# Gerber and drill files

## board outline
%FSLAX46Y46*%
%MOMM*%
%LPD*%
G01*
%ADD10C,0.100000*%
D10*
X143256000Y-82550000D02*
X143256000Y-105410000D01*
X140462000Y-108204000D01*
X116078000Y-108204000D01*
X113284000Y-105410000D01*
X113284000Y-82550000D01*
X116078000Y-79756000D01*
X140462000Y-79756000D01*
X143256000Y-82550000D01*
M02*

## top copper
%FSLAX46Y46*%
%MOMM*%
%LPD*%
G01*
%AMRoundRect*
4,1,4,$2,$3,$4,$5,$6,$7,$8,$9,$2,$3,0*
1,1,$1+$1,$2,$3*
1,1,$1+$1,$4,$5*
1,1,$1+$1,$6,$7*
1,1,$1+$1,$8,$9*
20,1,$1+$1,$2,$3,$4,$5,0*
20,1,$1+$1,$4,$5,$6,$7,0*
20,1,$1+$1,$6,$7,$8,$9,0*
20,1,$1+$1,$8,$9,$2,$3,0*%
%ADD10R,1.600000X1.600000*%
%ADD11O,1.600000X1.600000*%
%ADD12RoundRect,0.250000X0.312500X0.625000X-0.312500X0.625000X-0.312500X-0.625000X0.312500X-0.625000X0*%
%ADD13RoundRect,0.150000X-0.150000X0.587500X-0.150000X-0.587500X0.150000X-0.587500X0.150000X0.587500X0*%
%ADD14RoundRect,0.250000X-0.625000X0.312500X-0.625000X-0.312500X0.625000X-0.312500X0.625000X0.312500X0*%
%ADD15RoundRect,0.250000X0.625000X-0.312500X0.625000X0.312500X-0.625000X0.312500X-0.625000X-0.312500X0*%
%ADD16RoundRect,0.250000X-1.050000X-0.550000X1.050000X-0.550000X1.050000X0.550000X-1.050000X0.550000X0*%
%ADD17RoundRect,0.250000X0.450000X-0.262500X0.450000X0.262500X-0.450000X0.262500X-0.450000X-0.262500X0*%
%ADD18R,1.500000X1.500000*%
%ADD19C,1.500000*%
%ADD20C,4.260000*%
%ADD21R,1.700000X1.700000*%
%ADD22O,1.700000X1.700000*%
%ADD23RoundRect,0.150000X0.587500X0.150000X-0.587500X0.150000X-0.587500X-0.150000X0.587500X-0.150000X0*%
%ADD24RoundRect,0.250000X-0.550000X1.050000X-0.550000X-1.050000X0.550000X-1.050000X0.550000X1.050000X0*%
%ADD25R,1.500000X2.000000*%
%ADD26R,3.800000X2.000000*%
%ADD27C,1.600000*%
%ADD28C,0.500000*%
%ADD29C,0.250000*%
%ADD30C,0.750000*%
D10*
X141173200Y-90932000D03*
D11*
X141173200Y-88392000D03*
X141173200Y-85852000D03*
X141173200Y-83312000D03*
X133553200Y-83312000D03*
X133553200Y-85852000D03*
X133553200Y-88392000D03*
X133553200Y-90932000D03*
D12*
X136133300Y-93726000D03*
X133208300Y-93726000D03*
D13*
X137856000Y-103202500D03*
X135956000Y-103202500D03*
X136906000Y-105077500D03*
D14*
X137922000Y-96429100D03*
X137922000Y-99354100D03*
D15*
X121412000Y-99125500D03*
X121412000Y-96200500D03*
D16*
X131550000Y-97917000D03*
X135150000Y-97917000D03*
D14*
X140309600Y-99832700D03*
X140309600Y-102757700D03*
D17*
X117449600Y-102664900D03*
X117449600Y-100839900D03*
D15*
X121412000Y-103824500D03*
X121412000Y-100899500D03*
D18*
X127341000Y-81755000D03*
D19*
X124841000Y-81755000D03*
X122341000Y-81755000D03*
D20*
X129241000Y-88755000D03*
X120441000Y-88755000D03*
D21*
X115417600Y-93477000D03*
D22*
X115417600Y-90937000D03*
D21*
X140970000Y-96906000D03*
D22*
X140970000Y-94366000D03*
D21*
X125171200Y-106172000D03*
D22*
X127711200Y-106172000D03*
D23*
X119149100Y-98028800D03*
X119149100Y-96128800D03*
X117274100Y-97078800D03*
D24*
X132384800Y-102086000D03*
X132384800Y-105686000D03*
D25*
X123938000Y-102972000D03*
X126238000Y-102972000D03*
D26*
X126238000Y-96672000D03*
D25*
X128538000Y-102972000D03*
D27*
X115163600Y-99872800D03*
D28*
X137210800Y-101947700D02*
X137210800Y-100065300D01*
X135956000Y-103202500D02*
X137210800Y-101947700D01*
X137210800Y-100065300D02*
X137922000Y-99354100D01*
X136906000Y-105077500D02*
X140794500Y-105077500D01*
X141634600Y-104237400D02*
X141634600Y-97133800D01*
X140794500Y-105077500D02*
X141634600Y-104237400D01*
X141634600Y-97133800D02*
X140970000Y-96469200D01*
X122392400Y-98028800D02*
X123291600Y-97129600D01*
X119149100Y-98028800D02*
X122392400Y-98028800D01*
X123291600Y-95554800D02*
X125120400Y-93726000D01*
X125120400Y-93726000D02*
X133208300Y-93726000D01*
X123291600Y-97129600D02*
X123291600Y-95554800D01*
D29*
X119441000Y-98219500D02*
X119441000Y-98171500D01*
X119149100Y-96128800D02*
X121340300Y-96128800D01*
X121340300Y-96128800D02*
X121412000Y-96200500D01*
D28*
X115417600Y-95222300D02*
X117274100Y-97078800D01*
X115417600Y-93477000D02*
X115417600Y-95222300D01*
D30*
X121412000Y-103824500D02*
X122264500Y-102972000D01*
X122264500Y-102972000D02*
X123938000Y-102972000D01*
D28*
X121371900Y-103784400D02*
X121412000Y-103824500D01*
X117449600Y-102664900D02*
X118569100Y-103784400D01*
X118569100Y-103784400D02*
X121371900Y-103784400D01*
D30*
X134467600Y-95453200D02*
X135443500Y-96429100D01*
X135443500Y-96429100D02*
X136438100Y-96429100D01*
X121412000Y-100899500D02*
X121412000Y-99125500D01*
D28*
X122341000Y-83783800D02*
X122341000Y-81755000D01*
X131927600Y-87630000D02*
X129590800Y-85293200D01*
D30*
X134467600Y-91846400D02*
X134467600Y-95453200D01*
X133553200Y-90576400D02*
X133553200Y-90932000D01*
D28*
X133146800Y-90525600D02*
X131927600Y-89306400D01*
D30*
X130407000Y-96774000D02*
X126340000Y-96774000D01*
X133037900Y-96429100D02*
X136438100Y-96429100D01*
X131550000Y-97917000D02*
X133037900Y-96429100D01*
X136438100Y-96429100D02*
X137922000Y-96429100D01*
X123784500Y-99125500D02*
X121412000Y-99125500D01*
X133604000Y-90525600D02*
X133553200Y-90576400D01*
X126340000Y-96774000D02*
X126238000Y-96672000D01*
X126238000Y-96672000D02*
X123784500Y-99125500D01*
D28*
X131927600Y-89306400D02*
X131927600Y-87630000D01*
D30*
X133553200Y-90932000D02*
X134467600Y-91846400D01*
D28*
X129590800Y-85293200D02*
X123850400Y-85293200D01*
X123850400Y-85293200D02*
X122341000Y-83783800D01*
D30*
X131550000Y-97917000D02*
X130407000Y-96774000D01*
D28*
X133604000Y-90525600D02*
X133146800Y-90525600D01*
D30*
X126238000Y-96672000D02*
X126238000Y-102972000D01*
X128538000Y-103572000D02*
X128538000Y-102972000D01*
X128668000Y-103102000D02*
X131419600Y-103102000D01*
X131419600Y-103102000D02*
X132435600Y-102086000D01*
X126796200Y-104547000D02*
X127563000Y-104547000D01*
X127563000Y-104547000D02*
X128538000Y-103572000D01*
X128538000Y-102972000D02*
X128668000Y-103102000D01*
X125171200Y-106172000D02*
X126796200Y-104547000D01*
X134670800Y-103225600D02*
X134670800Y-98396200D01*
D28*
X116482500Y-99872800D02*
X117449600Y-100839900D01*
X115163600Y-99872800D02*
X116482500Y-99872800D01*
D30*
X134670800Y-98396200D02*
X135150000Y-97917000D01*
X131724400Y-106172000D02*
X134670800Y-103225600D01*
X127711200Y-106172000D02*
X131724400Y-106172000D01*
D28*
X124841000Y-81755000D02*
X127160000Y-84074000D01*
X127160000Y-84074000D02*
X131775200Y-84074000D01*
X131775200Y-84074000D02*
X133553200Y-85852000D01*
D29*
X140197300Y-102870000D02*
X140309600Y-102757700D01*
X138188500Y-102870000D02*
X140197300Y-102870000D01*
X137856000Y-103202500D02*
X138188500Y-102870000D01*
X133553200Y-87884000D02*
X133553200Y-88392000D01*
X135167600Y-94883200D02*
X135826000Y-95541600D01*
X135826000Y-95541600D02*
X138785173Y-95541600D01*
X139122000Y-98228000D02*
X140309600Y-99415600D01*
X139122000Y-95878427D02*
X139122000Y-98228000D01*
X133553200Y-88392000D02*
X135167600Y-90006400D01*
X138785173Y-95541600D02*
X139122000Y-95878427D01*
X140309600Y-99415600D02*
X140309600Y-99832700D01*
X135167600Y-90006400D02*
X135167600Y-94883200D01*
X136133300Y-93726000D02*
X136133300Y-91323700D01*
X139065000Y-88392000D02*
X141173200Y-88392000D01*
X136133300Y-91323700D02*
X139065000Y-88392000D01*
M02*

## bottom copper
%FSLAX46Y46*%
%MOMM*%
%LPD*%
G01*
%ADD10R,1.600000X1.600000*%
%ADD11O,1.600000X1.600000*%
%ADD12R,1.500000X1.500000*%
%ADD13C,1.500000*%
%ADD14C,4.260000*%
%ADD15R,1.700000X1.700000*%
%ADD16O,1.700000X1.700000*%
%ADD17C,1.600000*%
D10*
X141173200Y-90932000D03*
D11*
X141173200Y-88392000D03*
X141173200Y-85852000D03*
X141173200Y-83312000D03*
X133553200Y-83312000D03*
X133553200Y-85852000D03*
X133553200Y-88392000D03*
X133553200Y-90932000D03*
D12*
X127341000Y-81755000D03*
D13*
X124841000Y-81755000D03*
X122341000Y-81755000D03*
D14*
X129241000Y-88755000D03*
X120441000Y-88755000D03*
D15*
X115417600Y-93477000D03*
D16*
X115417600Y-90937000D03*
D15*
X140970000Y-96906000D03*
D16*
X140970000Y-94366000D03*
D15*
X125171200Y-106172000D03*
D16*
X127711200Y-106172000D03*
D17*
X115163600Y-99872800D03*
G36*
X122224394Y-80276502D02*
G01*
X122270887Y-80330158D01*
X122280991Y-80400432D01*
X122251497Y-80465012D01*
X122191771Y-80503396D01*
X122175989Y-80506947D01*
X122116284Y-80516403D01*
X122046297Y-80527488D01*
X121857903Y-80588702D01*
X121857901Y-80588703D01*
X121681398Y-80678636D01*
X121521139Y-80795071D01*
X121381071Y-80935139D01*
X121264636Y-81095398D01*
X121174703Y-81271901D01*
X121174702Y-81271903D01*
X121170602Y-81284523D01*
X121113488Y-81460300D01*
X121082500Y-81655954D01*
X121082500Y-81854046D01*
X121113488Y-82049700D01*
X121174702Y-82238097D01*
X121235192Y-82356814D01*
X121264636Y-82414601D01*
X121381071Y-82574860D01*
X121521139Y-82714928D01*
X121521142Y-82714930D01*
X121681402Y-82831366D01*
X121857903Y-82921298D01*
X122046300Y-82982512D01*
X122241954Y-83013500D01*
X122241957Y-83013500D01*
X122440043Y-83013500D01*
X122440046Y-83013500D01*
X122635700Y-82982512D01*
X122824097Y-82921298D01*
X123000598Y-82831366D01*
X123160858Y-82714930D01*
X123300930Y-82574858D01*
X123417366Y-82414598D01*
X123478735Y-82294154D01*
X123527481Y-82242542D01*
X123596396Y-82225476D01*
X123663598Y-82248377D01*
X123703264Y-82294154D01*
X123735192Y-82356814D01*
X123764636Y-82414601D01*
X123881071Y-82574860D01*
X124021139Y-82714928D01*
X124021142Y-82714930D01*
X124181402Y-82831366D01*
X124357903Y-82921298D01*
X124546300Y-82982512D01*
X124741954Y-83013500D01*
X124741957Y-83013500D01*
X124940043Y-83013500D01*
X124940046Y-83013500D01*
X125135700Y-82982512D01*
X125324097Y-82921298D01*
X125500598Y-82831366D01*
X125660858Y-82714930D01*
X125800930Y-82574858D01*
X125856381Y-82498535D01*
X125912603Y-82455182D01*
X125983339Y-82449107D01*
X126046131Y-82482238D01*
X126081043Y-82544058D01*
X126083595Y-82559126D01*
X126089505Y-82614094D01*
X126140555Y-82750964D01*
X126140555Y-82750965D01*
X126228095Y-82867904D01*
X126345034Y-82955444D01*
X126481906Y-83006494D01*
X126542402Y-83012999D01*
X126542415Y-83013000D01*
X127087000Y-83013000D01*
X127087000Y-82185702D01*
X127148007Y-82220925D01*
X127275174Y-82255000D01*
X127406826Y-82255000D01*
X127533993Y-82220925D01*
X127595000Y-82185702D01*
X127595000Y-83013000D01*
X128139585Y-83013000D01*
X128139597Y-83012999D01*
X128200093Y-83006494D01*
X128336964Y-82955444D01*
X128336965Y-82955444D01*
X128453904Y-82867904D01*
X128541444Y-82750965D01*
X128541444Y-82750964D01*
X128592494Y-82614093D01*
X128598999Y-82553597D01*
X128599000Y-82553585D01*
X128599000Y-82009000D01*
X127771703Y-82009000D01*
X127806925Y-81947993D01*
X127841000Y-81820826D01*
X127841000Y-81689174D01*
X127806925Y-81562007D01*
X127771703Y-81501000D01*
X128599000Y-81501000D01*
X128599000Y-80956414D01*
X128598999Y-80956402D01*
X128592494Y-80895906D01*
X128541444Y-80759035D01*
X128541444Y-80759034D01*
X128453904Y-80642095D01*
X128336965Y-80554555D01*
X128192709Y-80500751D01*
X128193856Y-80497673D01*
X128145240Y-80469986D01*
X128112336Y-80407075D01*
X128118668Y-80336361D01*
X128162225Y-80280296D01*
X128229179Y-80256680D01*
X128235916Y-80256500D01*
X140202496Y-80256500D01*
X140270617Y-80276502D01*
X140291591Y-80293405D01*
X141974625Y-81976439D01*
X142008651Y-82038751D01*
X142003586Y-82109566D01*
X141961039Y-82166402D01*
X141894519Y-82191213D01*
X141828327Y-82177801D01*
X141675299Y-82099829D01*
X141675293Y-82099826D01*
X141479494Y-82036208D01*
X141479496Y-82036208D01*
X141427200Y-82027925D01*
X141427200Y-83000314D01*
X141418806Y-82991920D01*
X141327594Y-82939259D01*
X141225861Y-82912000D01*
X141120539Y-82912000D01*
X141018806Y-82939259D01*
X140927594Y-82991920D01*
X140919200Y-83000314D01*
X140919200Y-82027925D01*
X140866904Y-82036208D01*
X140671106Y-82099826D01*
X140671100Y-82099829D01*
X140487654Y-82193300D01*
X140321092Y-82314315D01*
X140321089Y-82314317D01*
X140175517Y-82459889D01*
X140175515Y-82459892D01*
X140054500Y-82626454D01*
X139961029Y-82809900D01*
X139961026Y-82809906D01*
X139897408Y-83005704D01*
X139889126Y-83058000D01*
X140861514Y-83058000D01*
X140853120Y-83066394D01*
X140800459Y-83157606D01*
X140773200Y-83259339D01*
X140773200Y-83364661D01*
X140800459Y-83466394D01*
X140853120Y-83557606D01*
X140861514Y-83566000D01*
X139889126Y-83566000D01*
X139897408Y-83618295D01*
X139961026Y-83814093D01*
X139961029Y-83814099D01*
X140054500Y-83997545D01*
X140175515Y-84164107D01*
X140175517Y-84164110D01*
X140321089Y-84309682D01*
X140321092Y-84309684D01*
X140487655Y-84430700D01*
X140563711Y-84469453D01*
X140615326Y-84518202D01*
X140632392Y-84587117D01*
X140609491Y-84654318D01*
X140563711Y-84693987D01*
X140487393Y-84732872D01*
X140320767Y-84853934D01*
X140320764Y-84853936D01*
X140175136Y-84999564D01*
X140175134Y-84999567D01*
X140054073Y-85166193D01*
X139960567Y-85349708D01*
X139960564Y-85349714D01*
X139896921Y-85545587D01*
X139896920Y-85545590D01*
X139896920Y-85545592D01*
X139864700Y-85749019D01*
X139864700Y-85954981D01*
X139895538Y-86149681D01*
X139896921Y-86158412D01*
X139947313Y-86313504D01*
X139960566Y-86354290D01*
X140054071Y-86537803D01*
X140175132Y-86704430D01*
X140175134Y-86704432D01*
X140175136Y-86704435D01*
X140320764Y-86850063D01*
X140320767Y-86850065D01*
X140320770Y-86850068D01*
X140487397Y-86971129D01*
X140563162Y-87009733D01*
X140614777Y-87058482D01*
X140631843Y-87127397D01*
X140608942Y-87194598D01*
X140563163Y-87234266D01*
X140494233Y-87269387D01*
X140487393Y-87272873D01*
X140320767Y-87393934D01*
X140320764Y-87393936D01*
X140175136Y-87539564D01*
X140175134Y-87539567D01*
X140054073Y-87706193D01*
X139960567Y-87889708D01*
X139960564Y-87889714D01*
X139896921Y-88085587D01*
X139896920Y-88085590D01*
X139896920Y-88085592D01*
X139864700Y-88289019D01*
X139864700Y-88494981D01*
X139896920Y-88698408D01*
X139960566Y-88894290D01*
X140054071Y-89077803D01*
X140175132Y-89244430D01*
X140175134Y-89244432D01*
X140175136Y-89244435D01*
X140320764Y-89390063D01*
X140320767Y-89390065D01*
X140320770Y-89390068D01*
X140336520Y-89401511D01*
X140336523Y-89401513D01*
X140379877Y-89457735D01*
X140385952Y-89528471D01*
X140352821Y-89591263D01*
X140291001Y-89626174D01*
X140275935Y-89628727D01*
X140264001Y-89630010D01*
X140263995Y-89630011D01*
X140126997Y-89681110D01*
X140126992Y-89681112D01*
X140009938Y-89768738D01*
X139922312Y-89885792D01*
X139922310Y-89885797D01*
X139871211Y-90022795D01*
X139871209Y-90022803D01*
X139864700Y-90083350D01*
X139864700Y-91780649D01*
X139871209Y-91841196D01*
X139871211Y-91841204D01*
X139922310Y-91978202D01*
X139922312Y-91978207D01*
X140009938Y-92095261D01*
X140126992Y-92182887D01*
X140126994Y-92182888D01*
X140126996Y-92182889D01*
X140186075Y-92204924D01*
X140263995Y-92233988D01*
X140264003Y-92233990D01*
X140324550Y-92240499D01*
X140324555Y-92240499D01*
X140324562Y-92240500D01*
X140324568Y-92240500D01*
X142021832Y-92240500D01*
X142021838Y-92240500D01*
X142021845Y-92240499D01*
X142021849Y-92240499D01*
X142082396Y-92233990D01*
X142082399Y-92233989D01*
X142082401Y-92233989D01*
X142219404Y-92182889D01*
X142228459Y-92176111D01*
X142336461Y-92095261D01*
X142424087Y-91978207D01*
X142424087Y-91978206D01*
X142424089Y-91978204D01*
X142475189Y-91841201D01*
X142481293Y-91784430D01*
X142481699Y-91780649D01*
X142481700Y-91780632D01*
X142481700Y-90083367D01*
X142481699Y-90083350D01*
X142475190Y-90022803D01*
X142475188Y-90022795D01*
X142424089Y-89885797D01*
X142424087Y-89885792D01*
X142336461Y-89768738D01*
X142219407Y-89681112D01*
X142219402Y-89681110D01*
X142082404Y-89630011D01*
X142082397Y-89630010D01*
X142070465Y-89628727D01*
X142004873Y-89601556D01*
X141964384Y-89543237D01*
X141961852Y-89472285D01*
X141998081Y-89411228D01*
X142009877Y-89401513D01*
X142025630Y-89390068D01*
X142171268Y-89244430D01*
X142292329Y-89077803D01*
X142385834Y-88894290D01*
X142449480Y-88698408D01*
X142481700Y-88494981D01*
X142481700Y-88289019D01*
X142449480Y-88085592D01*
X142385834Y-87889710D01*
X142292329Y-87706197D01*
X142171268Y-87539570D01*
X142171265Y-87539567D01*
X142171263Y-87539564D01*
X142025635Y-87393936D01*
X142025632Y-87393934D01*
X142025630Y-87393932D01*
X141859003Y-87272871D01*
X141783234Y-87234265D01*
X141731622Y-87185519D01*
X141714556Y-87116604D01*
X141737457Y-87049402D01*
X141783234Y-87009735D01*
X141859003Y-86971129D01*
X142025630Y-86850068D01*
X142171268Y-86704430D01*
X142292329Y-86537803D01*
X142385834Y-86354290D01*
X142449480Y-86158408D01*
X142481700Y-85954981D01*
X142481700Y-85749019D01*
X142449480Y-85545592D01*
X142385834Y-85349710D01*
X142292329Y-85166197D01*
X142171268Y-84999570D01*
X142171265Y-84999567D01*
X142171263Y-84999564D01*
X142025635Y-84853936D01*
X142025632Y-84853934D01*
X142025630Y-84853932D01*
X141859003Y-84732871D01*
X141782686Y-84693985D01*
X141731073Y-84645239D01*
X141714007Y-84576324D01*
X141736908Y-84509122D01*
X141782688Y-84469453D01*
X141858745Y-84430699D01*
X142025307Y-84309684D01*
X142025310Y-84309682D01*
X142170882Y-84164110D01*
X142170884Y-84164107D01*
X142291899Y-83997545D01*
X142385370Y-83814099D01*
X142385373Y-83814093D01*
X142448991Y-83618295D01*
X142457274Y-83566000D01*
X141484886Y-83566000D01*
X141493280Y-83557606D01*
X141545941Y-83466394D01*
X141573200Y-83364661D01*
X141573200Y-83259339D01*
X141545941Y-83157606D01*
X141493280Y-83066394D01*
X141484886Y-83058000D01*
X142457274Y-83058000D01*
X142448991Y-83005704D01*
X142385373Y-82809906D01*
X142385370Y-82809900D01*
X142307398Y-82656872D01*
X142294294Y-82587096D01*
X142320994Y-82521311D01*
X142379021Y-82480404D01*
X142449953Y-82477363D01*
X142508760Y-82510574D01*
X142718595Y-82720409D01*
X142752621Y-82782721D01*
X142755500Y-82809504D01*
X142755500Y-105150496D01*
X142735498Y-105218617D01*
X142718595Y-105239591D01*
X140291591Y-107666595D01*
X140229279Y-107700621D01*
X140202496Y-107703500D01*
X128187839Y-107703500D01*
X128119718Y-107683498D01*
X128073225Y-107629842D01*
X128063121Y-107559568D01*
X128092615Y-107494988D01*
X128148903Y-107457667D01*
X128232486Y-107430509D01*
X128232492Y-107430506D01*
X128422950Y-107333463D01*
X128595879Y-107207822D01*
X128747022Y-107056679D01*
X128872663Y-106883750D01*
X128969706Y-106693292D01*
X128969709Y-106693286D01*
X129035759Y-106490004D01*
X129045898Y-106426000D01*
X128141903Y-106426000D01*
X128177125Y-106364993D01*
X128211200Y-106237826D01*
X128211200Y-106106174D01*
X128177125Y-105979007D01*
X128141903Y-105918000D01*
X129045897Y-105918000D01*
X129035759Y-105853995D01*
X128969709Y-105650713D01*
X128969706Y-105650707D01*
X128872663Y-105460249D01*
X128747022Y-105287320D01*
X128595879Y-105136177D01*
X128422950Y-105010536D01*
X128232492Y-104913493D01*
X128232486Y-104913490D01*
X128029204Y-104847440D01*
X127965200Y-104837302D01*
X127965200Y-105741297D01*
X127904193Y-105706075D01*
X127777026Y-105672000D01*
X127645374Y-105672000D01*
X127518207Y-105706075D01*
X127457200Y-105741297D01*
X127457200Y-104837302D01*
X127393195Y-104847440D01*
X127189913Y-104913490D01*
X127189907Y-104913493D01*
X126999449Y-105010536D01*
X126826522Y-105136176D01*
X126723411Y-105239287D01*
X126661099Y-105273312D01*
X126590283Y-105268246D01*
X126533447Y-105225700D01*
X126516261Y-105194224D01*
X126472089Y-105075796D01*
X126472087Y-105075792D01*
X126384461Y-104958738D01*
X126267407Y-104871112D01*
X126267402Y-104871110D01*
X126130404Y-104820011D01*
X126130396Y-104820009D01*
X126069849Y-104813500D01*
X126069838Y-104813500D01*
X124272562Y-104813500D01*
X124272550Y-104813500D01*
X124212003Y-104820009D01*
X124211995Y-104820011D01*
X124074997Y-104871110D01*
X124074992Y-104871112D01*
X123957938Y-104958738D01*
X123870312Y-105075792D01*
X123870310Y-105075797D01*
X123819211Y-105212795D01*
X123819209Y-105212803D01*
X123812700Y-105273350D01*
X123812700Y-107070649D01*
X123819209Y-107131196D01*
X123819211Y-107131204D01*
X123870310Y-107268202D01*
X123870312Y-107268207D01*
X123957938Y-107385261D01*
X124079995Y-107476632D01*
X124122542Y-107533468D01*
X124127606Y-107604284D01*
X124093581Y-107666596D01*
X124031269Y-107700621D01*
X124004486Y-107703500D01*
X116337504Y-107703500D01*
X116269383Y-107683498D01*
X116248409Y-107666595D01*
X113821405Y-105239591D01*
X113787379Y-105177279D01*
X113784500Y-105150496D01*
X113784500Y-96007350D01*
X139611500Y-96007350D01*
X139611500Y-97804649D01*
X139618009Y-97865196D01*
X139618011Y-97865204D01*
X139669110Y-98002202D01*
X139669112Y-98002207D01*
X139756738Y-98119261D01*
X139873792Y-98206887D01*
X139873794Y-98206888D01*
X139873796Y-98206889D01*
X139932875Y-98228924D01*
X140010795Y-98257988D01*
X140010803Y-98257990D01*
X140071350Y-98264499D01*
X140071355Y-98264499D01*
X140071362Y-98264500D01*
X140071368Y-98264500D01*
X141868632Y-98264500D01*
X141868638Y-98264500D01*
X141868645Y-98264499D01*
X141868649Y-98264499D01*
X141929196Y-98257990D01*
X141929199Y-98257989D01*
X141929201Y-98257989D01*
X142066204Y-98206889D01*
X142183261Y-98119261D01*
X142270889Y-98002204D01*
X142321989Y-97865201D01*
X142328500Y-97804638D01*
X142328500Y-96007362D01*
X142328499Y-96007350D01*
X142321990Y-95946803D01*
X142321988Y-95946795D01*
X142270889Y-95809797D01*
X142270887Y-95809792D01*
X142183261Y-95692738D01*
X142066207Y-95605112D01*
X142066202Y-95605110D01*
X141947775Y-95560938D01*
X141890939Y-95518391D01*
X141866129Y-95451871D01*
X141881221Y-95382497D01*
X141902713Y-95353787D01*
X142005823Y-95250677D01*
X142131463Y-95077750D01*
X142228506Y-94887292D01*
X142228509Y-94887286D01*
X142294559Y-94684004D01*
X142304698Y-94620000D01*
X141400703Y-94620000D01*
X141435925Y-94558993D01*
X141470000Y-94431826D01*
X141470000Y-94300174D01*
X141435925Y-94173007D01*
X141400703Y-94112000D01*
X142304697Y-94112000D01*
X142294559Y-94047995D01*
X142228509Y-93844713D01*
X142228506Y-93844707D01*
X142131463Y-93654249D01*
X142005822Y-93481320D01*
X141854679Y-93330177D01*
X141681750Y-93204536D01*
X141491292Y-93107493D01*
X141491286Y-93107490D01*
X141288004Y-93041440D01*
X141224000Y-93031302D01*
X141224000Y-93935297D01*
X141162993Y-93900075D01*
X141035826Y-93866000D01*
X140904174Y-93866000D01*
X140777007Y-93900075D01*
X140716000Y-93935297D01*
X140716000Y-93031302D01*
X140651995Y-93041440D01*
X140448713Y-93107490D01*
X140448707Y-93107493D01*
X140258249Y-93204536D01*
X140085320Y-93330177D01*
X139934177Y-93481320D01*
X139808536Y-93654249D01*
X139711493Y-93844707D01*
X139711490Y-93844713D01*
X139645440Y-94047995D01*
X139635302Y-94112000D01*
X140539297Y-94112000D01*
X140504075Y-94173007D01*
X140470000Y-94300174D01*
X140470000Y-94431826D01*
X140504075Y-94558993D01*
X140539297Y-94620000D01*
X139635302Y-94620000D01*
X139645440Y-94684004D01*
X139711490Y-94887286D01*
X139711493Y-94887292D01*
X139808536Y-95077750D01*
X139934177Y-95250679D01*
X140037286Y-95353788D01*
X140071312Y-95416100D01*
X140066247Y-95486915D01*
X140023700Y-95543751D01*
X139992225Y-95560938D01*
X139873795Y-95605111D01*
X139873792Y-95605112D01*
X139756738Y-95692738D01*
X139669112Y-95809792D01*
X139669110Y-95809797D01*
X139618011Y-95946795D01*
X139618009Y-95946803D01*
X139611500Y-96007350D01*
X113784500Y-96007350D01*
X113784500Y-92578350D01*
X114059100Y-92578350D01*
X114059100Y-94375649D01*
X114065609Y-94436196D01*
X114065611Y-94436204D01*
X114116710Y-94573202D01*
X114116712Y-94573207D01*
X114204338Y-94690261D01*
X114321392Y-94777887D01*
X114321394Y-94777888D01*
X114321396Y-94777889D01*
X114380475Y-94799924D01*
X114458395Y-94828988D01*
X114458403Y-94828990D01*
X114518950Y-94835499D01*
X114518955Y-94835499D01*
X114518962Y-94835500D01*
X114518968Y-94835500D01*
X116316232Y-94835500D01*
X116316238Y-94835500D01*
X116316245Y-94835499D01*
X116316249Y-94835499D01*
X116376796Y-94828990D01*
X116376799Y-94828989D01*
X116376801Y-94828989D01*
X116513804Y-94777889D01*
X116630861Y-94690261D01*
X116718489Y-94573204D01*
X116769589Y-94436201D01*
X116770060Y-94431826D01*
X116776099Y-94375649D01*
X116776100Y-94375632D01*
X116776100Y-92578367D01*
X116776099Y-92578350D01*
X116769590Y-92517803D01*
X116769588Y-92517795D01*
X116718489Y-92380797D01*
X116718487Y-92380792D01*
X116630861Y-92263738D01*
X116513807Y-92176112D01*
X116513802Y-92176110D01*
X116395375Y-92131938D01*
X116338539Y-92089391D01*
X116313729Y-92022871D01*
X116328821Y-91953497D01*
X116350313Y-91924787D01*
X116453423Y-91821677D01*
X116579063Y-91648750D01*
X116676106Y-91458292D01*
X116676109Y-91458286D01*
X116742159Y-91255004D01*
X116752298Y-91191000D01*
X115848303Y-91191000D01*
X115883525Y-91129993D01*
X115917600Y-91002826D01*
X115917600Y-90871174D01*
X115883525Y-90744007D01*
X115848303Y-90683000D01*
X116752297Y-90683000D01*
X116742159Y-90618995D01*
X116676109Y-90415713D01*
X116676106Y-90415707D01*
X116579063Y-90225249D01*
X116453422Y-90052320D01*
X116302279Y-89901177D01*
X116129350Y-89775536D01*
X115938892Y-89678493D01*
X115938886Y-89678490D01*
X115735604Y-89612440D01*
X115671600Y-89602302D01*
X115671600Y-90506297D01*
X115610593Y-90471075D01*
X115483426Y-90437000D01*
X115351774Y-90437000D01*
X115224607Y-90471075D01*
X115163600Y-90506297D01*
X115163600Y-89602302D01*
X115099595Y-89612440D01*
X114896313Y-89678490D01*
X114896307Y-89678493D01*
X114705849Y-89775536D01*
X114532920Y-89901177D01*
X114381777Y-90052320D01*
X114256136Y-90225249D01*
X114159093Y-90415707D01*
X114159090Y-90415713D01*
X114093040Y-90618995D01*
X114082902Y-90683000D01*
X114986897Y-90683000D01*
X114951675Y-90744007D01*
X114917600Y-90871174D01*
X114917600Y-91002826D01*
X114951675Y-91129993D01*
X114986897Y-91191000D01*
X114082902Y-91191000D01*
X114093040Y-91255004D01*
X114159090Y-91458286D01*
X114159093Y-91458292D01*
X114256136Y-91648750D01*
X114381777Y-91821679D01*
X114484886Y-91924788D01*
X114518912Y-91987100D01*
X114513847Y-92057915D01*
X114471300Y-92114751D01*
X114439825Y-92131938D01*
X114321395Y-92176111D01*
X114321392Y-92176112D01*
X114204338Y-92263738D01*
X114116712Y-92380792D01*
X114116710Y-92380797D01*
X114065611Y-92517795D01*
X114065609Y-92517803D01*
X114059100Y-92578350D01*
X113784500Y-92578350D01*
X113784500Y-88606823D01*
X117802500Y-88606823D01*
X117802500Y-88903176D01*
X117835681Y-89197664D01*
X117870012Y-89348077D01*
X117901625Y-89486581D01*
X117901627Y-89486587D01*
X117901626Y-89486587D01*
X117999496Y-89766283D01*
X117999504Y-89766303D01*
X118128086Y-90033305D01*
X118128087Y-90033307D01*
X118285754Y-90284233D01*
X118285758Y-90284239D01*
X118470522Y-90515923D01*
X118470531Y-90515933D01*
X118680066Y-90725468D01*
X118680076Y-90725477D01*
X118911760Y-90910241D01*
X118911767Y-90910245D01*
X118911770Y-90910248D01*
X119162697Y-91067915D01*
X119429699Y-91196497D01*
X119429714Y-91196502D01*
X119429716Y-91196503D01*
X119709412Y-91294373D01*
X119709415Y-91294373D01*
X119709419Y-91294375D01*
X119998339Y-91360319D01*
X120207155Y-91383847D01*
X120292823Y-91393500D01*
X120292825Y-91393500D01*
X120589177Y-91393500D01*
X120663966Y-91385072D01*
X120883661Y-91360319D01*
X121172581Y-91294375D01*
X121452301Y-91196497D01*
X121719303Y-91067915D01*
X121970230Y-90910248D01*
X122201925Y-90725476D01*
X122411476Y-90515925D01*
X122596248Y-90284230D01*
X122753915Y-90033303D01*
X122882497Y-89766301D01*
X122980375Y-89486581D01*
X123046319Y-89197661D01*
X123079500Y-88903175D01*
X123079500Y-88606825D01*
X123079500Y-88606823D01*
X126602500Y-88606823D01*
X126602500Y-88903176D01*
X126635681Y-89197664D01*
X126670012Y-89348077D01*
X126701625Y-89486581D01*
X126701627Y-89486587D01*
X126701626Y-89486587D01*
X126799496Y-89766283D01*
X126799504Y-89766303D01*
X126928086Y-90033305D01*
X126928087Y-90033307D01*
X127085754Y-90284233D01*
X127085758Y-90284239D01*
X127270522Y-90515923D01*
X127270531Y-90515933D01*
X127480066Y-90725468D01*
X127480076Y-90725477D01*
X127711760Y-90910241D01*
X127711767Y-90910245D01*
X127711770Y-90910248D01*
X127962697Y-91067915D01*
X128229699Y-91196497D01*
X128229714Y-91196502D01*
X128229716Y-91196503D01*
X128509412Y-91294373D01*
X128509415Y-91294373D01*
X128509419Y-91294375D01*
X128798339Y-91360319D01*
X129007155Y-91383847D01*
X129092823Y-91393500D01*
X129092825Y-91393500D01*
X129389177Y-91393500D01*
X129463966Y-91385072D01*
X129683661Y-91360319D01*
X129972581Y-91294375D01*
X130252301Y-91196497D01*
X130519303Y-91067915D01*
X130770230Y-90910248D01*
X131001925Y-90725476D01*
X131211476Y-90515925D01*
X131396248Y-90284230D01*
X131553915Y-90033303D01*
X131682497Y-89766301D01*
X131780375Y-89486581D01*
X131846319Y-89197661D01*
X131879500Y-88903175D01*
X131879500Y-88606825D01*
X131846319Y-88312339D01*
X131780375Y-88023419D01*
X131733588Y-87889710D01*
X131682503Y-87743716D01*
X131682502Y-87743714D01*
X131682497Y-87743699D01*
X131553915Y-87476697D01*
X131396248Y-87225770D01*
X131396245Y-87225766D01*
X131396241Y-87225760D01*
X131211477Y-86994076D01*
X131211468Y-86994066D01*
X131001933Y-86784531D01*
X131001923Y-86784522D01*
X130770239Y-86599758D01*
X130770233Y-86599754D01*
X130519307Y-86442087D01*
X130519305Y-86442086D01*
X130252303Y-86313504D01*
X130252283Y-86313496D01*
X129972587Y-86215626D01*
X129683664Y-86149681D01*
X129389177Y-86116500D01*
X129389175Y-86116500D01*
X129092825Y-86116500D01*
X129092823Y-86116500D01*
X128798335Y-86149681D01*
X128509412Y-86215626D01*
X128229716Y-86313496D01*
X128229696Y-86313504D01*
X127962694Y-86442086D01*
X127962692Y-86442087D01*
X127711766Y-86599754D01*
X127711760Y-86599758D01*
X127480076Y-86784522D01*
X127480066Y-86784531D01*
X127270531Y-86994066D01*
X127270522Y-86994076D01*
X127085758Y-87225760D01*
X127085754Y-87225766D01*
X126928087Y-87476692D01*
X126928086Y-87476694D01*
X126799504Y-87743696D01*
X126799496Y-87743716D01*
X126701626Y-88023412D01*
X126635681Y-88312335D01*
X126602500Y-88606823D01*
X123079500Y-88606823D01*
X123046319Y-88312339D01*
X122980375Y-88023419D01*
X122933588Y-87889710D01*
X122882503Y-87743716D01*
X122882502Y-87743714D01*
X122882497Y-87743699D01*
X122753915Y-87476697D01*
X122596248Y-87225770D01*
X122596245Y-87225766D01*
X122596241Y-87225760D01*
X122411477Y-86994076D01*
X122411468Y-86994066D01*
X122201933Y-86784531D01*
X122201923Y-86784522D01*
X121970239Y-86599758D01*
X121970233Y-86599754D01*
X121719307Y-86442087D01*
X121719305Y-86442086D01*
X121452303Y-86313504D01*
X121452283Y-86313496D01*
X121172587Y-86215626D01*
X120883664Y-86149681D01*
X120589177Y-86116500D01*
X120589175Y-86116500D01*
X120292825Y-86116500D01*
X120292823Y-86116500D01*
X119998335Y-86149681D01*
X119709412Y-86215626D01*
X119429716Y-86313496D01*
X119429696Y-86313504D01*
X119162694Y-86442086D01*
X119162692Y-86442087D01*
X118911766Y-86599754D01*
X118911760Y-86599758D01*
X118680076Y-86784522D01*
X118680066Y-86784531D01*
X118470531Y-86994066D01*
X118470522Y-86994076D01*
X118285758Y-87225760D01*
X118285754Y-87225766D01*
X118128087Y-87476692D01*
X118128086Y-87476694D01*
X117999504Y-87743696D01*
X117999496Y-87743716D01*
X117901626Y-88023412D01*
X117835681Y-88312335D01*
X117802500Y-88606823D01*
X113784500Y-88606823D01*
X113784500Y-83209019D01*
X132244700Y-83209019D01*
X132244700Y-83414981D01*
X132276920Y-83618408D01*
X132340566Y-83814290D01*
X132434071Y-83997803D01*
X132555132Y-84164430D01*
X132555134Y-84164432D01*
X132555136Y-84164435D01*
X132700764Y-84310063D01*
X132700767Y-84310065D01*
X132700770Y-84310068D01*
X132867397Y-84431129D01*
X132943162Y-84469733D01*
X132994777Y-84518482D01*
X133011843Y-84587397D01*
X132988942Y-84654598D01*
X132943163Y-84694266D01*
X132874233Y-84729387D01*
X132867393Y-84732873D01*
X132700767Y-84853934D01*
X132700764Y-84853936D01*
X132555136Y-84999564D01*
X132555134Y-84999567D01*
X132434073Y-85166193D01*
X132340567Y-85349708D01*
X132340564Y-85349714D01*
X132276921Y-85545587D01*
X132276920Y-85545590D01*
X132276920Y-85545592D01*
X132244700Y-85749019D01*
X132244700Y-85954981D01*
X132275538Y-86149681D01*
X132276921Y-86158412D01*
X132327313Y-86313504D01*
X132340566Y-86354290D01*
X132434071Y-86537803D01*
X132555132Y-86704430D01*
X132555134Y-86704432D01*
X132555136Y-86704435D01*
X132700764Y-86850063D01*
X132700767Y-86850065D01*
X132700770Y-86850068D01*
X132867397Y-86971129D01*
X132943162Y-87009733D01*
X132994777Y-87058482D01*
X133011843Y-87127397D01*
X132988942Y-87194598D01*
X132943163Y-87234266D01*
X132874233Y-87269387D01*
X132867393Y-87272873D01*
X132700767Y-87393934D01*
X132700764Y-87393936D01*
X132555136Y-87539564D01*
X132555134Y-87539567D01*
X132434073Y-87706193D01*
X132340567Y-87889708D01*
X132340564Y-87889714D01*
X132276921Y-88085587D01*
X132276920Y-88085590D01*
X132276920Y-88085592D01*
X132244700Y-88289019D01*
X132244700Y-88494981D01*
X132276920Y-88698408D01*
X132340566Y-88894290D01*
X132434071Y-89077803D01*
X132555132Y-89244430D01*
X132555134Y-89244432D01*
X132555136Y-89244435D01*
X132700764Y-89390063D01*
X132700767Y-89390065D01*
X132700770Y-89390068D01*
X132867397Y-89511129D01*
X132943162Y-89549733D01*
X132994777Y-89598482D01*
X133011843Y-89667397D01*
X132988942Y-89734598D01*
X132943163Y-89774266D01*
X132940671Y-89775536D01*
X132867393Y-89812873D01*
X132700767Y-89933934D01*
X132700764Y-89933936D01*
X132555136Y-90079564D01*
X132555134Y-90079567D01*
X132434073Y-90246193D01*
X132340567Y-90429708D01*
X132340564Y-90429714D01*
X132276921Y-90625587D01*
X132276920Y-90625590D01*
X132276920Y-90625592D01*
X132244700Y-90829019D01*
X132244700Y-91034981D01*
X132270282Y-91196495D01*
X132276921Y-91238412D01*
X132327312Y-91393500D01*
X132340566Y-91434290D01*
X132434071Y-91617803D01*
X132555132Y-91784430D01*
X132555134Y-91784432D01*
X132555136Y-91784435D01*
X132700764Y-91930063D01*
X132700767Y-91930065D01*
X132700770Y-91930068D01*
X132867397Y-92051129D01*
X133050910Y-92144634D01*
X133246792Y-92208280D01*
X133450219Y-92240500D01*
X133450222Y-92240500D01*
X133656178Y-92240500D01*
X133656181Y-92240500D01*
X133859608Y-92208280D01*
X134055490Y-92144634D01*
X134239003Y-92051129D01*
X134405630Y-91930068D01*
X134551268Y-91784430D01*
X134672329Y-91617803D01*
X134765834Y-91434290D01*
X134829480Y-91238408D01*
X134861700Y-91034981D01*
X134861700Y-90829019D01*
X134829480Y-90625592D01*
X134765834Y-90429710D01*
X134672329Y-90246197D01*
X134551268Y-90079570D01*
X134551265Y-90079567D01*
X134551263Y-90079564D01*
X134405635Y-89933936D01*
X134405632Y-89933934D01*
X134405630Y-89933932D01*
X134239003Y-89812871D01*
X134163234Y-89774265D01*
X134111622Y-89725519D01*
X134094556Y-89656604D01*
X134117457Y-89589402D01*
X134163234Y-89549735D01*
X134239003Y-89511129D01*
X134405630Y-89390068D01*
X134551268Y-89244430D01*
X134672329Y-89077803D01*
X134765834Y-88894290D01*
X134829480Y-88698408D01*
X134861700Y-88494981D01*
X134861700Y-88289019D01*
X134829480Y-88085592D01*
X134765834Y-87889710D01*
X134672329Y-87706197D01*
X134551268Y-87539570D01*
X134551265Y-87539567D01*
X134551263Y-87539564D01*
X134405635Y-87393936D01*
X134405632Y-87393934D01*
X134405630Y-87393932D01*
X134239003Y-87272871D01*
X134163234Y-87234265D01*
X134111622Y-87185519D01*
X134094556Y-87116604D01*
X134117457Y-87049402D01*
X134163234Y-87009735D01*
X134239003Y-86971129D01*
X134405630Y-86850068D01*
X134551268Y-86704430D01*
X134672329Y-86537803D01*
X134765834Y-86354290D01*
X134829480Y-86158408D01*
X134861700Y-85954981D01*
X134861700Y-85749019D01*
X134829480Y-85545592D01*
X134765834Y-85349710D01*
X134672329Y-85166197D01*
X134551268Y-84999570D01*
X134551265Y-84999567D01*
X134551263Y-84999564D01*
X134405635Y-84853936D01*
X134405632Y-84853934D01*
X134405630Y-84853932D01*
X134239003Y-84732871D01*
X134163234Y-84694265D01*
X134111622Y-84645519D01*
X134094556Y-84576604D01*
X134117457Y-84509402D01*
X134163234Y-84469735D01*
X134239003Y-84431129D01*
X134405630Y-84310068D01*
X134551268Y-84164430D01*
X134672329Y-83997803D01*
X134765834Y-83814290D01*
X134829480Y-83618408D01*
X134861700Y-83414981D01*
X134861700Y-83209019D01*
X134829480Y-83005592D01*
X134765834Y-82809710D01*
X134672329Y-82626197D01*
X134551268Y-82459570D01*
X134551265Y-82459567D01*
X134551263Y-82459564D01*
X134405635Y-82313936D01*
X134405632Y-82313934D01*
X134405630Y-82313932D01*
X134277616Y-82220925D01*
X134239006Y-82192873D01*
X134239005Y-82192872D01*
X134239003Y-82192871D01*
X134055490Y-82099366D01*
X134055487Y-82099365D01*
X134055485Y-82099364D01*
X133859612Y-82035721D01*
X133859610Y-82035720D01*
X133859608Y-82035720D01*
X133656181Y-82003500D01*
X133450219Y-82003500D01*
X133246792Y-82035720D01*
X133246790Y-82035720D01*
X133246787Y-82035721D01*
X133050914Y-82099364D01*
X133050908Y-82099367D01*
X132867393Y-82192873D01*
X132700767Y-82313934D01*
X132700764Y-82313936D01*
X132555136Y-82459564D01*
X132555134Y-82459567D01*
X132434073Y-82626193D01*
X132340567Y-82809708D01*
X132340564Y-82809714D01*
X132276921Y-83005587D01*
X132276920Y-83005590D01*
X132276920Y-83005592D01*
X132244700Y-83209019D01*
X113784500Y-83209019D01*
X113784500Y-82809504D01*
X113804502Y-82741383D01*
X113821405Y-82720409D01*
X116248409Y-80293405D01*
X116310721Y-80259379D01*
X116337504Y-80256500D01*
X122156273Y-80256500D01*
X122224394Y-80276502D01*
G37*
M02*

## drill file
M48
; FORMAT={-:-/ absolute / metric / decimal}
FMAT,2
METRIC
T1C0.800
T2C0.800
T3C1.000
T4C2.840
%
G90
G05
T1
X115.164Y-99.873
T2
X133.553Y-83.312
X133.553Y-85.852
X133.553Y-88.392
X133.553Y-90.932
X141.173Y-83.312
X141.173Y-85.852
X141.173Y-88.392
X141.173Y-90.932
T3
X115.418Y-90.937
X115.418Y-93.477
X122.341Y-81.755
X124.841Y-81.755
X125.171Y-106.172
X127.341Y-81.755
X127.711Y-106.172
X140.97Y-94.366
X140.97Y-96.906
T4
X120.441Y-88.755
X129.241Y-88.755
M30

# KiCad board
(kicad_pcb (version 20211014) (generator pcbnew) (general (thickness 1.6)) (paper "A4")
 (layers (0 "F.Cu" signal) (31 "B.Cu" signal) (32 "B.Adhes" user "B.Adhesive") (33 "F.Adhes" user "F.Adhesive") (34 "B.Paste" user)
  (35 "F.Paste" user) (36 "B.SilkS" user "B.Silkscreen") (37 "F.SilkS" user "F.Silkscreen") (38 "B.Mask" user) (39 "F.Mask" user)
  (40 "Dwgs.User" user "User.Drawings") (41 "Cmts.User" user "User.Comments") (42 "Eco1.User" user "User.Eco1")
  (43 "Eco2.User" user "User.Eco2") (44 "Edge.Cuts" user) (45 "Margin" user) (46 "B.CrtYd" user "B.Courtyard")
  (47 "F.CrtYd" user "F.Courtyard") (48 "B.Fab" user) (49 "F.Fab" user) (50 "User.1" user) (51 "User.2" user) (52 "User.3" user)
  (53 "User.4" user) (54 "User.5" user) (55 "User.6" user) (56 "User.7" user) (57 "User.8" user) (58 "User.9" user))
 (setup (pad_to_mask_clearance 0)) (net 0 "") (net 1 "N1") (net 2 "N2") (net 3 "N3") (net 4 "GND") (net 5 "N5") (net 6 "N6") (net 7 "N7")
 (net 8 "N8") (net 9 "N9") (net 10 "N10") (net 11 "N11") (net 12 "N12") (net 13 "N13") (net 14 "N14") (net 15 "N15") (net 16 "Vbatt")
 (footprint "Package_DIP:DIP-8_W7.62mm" (layer "F.Cu") (at 141.1732 90.932 180)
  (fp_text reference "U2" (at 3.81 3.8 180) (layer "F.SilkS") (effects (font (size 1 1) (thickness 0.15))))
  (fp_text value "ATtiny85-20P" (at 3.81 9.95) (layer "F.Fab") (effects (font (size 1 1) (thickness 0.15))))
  (pad "1" thru_hole rect (at 0 0 180) (size 1.6 1.6) (drill 0.8) (layers *.Cu *.Mask) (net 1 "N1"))
  (pad "2" thru_hole oval (at 0 2.54 180) (size 1.6 1.6) (drill 0.8) (layers *.Cu *.Mask) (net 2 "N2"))
  (pad "3" thru_hole oval (at 0 5.08 180) (size 1.6 1.6) (drill 0.8) (layers *.Cu *.Mask) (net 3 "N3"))
  (pad "4" thru_hole oval (at 0 7.62 180) (size 1.6 1.6) (drill 0.8) (layers *.Cu *.Mask) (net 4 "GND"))
  (pad "5" thru_hole oval (at 7.62 7.62 180) (size 1.6 1.6) (drill 0.8) (layers *.Cu *.Mask) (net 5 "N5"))
  (pad "6" thru_hole oval (at 7.62 5.08 180) (size 1.6 1.6) (drill 0.8) (layers *.Cu *.Mask) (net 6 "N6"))
  (pad "7" thru_hole oval (at 7.62 2.54 180) (size 1.6 1.6) (drill 0.8) (layers *.Cu *.Mask) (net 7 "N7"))
  (pad "8" thru_hole oval (at 7.62 0 180) (size 1.6 1.6) (drill 0.8) (layers *.Cu *.Mask) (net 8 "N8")))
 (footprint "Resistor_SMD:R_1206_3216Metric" (layer "F.Cu") (at 134.6708 93.726 180)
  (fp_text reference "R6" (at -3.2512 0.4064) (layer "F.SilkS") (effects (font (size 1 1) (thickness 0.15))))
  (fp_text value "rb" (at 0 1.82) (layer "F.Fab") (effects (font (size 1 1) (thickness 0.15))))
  (pad "1" smd roundrect (at -1.4625 0 180) (size 1.125 1.75) (layers "F.Cu" "F.Paste" "F.Mask") (roundrect_rratio 0.2222222222)
   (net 2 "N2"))
  (pad "2" smd roundrect (at 1.4625 0 180) (size 1.125 1.75) (layers "F.Cu" "F.Paste" "F.Mask") (roundrect_rratio 0.2222222222) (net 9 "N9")))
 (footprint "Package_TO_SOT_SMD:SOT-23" (layer "F.Cu") (at 136.906 104.14 -90)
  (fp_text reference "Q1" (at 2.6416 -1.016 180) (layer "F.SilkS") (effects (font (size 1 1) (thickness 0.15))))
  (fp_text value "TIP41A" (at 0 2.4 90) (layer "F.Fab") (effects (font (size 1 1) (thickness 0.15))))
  (pad "1" smd roundrect (at -0.9375 -0.95 270) (size 1.475 0.6) (layers "F.Cu" "F.Paste" "F.Mask") (roundrect_rratio 0.25) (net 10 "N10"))
  (pad "2" smd roundrect (at -0.9375 0.95 270) (size 1.475 0.6) (layers "F.Cu" "F.Paste" "F.Mask") (roundrect_rratio 0.25) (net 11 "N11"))
  (pad "3" smd roundrect (at 0.9375 0 270) (size 1.475 0.6) (layers "F.Cu" "F.Paste" "F.Mask") (roundrect_rratio 0.25) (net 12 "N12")))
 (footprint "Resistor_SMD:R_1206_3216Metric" (layer "F.Cu") (at 137.922 97.8916 -90)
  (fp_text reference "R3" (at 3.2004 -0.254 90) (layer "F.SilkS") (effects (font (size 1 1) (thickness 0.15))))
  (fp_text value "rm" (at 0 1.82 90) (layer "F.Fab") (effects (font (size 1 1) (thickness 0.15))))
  (pad "1" smd roundrect (at -1.4625 0 270) (size 1.125 1.75) (layers "F.Cu" "F.Paste" "F.Mask") (roundrect_rratio 0.2222222222)
   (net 8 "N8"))
  (pad "2" smd roundrect (at 1.4625 0 270) (size 1.125 1.75) (layers "F.Cu" "F.Paste" "F.Mask") (roundrect_rratio 0.2222222222)
   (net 11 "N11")))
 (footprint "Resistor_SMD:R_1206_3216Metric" (layer "F.Cu") (at 121.412 97.663 90)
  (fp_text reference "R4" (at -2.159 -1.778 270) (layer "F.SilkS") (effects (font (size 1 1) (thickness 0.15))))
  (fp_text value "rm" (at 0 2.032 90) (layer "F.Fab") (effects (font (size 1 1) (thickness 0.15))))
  (pad "1" smd roundrect (at -1.4625 0 90) (size 1.125 1.75) (layers "F.Cu" "F.Paste" "F.Mask") (roundrect_rratio 0.2222222222) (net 8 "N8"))
  (pad "2" smd roundrect (at 1.4625 0 90) (size 1.125 1.75) (layers "F.Cu" "F.Paste" "F.Mask") (roundrect_rratio 0.2222222222)
   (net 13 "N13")))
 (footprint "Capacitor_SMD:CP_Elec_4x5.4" (layer "F.Cu") (at 133.35 97.917)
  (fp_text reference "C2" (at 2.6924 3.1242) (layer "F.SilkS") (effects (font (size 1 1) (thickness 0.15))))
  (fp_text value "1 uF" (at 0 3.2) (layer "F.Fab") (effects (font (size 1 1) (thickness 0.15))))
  (pad "1" smd roundrect (at -1.8 0) (size 2.6 1.6) (layers "F.Cu" "F.Paste" "F.Mask") (roundrect_rratio 0.15625) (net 8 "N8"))
  (pad "2" smd roundrect (at 1.8 0) (size 2.6 1.6) (layers "F.Cu" "F.Paste" "F.Mask") (roundrect_rratio 0.15625) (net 4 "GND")))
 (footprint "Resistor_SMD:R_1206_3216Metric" (layer "F.Cu") (at 140.3096 101.2952 -90)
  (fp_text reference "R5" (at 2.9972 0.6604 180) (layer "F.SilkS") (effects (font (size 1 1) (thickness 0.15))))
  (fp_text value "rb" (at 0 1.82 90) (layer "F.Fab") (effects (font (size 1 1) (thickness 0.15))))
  (pad "1" smd roundrect (at -1.4625 0 270) (size 1.125 1.75) (layers "F.Cu" "F.Paste" "F.Mask") (roundrect_rratio 0.2222222222)
   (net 7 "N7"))
  (pad "2" smd roundrect (at 1.4625 0 270) (size 1.125 1.75) (layers "F.Cu" "F.Paste" "F.Mask") (roundrect_rratio 0.2222222222)
   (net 10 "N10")))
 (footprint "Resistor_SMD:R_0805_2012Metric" (layer "F.Cu") (at 117.4496 101.7524 90)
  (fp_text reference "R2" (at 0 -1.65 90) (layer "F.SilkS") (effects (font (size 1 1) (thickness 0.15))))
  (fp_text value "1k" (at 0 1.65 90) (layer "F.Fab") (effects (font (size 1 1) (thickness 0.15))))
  (pad "1" smd roundrect (at -0.9125 0 90) (size 1.025 1.4) (layers "F.Cu" "F.Paste" "F.Mask") (roundrect_rratio 0.243902) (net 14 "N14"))
  (pad "2" smd roundrect (at 0.9125 0 90) (size 1.025 1.4) (layers "F.Cu" "F.Paste" "F.Mask") (roundrect_rratio 0.243902) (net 4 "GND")))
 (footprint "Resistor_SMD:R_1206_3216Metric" (layer "F.Cu") (at 121.412 102.362 90)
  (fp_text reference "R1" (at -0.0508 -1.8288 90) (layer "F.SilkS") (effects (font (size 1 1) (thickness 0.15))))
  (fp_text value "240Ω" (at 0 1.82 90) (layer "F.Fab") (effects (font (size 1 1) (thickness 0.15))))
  (pad "1" smd roundrect (at -1.4625 0 90) (size 1.125 1.75) (layers "F.Cu" "F.Paste" "F.Mask") (roundrect_rratio 0.2222222222)
   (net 14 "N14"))
  (pad "2" smd roundrect (at 1.4625 0 90) (size 1.125 1.75) (layers "F.Cu" "F.Paste" "F.Mask") (roundrect_rratio 0.2222222222) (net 8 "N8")))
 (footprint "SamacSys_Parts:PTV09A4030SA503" (layer "F.Cu") (at 127.341 81.755 180)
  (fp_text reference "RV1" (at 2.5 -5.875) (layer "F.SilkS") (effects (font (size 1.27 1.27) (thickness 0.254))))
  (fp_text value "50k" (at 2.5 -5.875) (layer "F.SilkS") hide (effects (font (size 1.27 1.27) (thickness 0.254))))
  (pad "1" thru_hole rect locked (at 0 0 180) (size 1.5 1.5) (drill 1) (layers *.Cu *.Mask) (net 4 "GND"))
  (pad "2" thru_hole circle locked (at 2.5 0 180) (size 1.5 1.5) (drill 1) (layers *.Cu *.Mask) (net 6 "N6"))
  (pad "3" thru_hole circle locked (at 5 0 180) (size 1.5 1.5) (drill 1) (layers *.Cu *.Mask) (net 8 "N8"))
  (pad "MH1" thru_hole circle locked (at -1.9 -7 180) (size 4.26 4.26) (drill 2.84) (layers *.Cu *.Mask))
  (pad "MH2" thru_hole circle locked (at 6.9 -7 180) (size 4.26 4.26) (drill 2.84) (layers *.Cu *.Mask)))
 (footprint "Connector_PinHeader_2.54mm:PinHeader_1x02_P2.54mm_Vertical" (layer "F.Cu") (at 115.4176 93.477 180)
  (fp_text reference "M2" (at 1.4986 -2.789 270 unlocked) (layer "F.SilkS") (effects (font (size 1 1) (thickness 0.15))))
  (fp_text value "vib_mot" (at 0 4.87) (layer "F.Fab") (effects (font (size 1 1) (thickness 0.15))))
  (pad "1" thru_hole rect (at 0 0 180) (size 1.7 1.7) (drill 1) (layers *.Cu *.Mask) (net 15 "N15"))
  (pad "2" thru_hole oval (at 0 2.54 180) (size 1.7 1.7) (drill 1) (layers *.Cu *.Mask) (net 4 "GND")))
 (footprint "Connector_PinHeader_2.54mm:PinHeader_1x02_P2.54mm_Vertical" (layer "F.Cu") (at 140.97 96.906 180)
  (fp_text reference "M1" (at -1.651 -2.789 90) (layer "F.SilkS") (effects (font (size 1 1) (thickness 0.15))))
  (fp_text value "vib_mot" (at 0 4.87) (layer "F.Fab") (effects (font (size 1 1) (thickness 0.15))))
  (pad "1" thru_hole rect (at 0 0 180) (size 1.7 1.7) (drill 1) (layers *.Cu *.Mask) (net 12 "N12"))
  (pad "2" thru_hole oval (at 0 2.54 180) (size 1.7 1.7) (drill 1) (layers *.Cu *.Mask) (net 4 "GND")))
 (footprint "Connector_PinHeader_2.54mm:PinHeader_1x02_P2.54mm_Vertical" (layer "F.Cu") (at 125.1712 106.172 90)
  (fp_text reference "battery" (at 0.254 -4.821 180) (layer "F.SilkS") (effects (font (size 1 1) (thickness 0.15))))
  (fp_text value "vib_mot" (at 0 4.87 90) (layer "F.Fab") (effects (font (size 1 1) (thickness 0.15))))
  (pad "1" thru_hole rect (at 0 0 90) (size 1.7 1.7) (drill 1) (layers *.Cu *.Mask) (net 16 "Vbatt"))
  (pad "2" thru_hole oval (at 0 2.54 90) (size 1.7 1.7) (drill 1) (layers *.Cu *.Mask) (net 4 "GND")))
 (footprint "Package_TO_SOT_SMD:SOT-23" (layer "F.Cu") (at 118.2116 97.0788 180)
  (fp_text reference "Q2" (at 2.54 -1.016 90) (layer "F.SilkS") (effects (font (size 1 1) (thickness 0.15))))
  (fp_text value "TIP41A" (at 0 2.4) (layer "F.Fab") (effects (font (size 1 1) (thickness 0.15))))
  (pad "1" smd roundrect (at -0.9375 -0.95 180) (size 1.475 0.6) (layers "F.Cu" "F.Paste" "F.Mask") (roundrect_rratio 0.25) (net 9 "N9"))
  (pad "2" smd roundrect (at -0.9375 0.95 180) (size 1.475 0.6) (layers "F.Cu" "F.Paste" "F.Mask") (roundrect_rratio 0.25) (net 13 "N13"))
  (pad "3" smd roundrect (at 0.9375 0 180) (size 1.475 0.6) (layers "F.Cu" "F.Paste" "F.Mask") (roundrect_rratio 0.25) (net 15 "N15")))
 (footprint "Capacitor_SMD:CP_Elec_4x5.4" (layer "F.Cu") (at 132.3848 103.886 -90)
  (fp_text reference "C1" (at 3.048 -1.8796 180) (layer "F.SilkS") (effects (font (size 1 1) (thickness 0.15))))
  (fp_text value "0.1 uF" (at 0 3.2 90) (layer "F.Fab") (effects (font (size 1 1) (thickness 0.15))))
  (pad "1" smd roundrect (at -1.8 0 270) (size 2.6 1.6) (layers "F.Cu" "F.Paste" "F.Mask") (roundrect_rratio 0.15625) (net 16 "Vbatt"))
  (pad "2" smd roundrect (at 1.8 0 270) (size 2.6 1.6) (layers "F.Cu" "F.Paste" "F.Mask") (roundrect_rratio 0.15625) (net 4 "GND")))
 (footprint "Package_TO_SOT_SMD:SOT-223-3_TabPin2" (layer "F.Cu") (at 126.238 99.822 90)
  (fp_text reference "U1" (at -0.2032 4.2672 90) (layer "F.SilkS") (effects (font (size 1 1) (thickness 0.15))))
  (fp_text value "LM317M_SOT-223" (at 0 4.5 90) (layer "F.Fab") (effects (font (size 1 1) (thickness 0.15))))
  (pad "1" smd rect (at -3.15 -2.3 90) (size 2 1.5) (layers "F.Cu" "F.Paste" "F.Mask") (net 14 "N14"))
  (pad "2" smd rect (at -3.15 0 90) (size 2 1.5) (layers "F.Cu" "F.Paste" "F.Mask") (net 8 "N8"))
  (pad "2" smd rect (at 3.15 0 90) (size 2 3.8) (layers "F.Cu" "F.Paste" "F.Mask") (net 8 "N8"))
  (pad "3" smd rect (at -3.15 2.3 90) (size 2 1.5) (layers "F.Cu" "F.Paste" "F.Mask") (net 16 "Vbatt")))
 (gr_poly
  (pts (xy 143.256 82.55) (xy 143.256 105.41) (xy 140.462 108.204) (xy 116.078 108.204) (xy 113.284 105.41) (xy 113.284 82.55)
   (xy 116.078 79.756) (xy 140.462 79.756))
  (layer "Edge.Cuts") (width 0.1) (fill none))
 (segment (start 137.2108 101.9477) (end 137.2108 100.0653) (width 0.5) (layer "F.Cu") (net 11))
 (segment (start 135.956 103.2025) (end 137.2108 101.9477) (width 0.5) (layer "F.Cu") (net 11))
 (segment (start 137.2108 100.0653) (end 137.922 99.3541) (width 0.5) (layer "F.Cu") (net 11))
 (segment (start 136.906 105.0775) (end 140.7945 105.0775) (width 0.5) (layer "F.Cu") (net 12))
 (segment (start 141.6346 104.2374) (end 141.6346 97.1338) (width 0.5) (layer "F.Cu") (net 12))
 (segment (start 140.7945 105.0775) (end 141.6346 104.2374) (width 0.5) (layer "F.Cu") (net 12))
 (segment (start 141.6346 97.1338) (end 140.97 96.4692) (width 0.5) (layer "F.Cu") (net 12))
 (segment (start 122.3924 98.0288) (end 123.2916 97.1296) (width 0.5) (layer "F.Cu") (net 9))
 (segment (start 119.1491 98.0288) (end 122.3924 98.0288) (width 0.5) (layer "F.Cu") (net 9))
 (segment (start 123.2916 95.5548) (end 125.1204 93.726) (width 0.5) (layer "F.Cu") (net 9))
 (segment (start 125.1204 93.726) (end 133.2083 93.726) (width 0.5) (layer "F.Cu") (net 9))
 (segment (start 123.2916 97.1296) (end 123.2916 95.5548) (width 0.5) (layer "F.Cu") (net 9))
 (segment (start 119.441 98.2195) (end 119.441 98.1715) (width 0.25) (layer "F.Cu") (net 9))
 (segment (start 119.1491 96.1288) (end 121.3403 96.1288) (width 0.25) (layer "F.Cu") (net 13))
 (segment (start 121.3403 96.1288) (end 121.412 96.2005) (width 0.25) (layer "F.Cu") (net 13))
 (segment (start 115.4176 95.2223) (end 117.2741 97.0788) (width 0.5) (layer "F.Cu") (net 15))
 (segment (start 115.4176 93.477) (end 115.4176 95.2223) (width 0.5) (layer "F.Cu") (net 15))
 (segment (start 121.412 103.8245) (end 122.2645 102.972) (width 0.75) (layer "F.Cu") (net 14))
 (segment (start 122.2645 102.972) (end 123.938 102.972) (width 0.75) (layer "F.Cu") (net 14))
 (segment (start 121.3719 103.7844) (end 121.412 103.8245) (width 0.5) (layer "F.Cu") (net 14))
 (segment (start 117.4496 102.6649) (end 118.5691 103.7844) (width 0.5) (layer "F.Cu") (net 14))
 (segment (start 118.5691 103.7844) (end 121.3719 103.7844) (width 0.5) (layer "F.Cu") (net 14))
 (segment (start 134.4676 95.4532) (end 135.4435 96.4291) (width 0.75) (layer "F.Cu") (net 8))
 (segment (start 135.4435 96.4291) (end 136.4381 96.4291) (width 0.75) (layer "F.Cu") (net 8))
 (segment (start 121.412 100.8995) (end 121.412 99.1255) (width 0.75) (layer "F.Cu") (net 8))
 (segment (start 122.341 83.7838) (end 122.341 81.755) (width 0.5) (layer "F.Cu") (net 8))
 (segment (start 131.9276 87.63) (end 129.5908 85.2932) (width 0.5) (layer "F.Cu") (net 8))
 (segment (start 134.4676 91.8464) (end 134.4676 95.4532) (width 0.75) (layer "F.Cu") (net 8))
 (segment (start 133.5532 90.5764) (end 133.5532 90.932) (width 0.75) (layer "F.Cu") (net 8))
 (segment (start 133.1468 90.5256) (end 131.9276 89.3064) (width 0.5) (layer "F.Cu") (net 8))
 (segment (start 130.407 96.774) (end 126.34 96.774) (width 0.75) (layer "F.Cu") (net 8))
 (segment (start 133.0379 96.4291) (end 136.4381 96.4291) (width 0.75) (layer "F.Cu") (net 8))
 (segment (start 131.55 97.917) (end 133.0379 96.4291) (width 0.75) (layer "F.Cu") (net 8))
 (segment (start 136.4381 96.4291) (end 137.922 96.4291) (width 0.75) (layer "F.Cu") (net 8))
 (segment (start 123.7845 99.1255) (end 121.412 99.1255) (width 0.75) (layer "F.Cu") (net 8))
 (segment (start 133.604 90.5256) (end 133.5532 90.5764) (width 0.75) (layer "F.Cu") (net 8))
 (segment (start 126.34 96.774) (end 126.238 96.672) (width 0.75) (layer "F.Cu") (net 8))
 (segment (start 126.238 96.672) (end 123.7845 99.1255) (width 0.75) (layer "F.Cu") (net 8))
 (segment (start 131.9276 89.3064) (end 131.9276 87.63) (width 0.5) (layer "F.Cu") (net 8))
 (segment (start 133.5532 90.932) (end 134.4676 91.8464) (width 0.75) (layer "F.Cu") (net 8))
 (segment (start 129.5908 85.2932) (end 123.8504 85.2932) (width 0.5) (layer "F.Cu") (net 8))
 (segment (start 123.8504 85.2932) (end 122.341 83.7838) (width 0.5) (layer "F.Cu") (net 8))
 (segment (start 131.55 97.917) (end 130.407 96.774) (width 0.75) (layer "F.Cu") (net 8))
 (segment (start 133.604 90.5256) (end 133.1468 90.5256) (width 0.5) (layer "F.Cu") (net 8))
 (segment (start 126.238 96.672) (end 126.238 102.972) (width 0.75) (layer "F.Cu") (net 8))
 (segment (start 128.538 103.572) (end 128.538 102.972) (width 0.75) (layer "F.Cu") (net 16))
 (segment (start 128.668 103.102) (end 131.4196 103.102) (width 0.75) (layer "F.Cu") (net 16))
 (segment (start 131.4196 103.102) (end 132.4356 102.086) (width 0.75) (layer "F.Cu") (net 16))
 (segment (start 126.7962 104.547) (end 127.563 104.547) (width 0.75) (layer "F.Cu") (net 16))
 (segment (start 127.563 104.547) (end 128.538 103.572) (width 0.75) (layer "F.Cu") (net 16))
 (segment (start 128.538 102.972) (end 128.668 103.102) (width 0.75) (layer "F.Cu") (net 16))
 (segment (start 125.1712 106.172) (end 126.7962 104.547) (width 0.75) (layer "F.Cu") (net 16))
 (segment (start 134.6708 103.2256) (end 134.6708 98.3962) (width 0.75) (layer "F.Cu") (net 4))
 (segment (start 116.4825 99.8728) (end 117.4496 100.8399) (width 0.5) (layer "F.Cu") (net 4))
 (segment (start 115.1636 99.8728) (end 116.4825 99.8728) (width 0.5) (layer "F.Cu") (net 4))
 (segment (start 134.6708 98.3962) (end 135.15 97.917) (width 0.75) (layer "F.Cu") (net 4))
 (segment (start 131.7244 106.172) (end 134.6708 103.2256) (width 0.75) (layer "F.Cu") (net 4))
 (segment (start 127.7112 106.172) (end 131.7244 106.172) (width 0.75) (layer "F.Cu") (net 4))
 (via (at 115.1636 99.8728) (size 1.6) (drill 0.8) (layers "F.Cu" "B.Cu") (free) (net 4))
 (segment (start 124.841 81.755) (end 127.16 84.074) (width 0.5) (layer "F.Cu") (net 6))
 (segment (start 127.16 84.074) (end 131.7752 84.074) (width 0.5) (layer "F.Cu") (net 6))
 (segment (start 131.7752 84.074) (end 133.5532 85.852) (width 0.5) (layer "F.Cu") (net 6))
 (segment (start 140.1973 102.87) (end 140.3096 102.7577) (width 0.25) (layer "F.Cu") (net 10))
 (segment (start 138.1885 102.87) (end 140.1973 102.87) (width 0.25) (layer "F.Cu") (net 10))
 (segment (start 137.856 103.2025) (end 138.1885 102.87) (width 0.25) (layer "F.Cu") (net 10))
 (segment (start 133.5532 87.884) (end 133.5532 88.392) (width 0.25) (layer "F.Cu") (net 7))
 (segment (start 135.1676 94.8832) (end 135.826 95.5416) (width 0.25) (layer "F.Cu") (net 7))
 (segment (start 135.826 95.5416) (end 138.785173 95.5416) (width 0.25) (layer "F.Cu") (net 7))
 (segment (start 139.122 98.228) (end 140.3096 99.4156) (width 0.25) (layer "F.Cu") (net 7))
 (segment (start 139.122 95.878427) (end 139.122 98.228) (width 0.25) (layer "F.Cu") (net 7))
 (segment (start 133.5532 88.392) (end 135.1676 90.0064) (width 0.25) (layer "F.Cu") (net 7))
 (segment (start 138.785173 95.5416) (end 139.122 95.878427) (width 0.25) (layer "F.Cu") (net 7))
 (segment (start 140.3096 99.4156) (end 140.3096 99.8327) (width 0.25) (layer "F.Cu") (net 7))
 (segment (start 135.1676 90.0064) (end 135.1676 94.8832) (width 0.25) (layer "F.Cu") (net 7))
 (segment (start 136.1333 93.726) (end 136.1333 91.3237) (width 0.25) (layer "F.Cu") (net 2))
 (segment (start 139.065 88.392) (end 141.1732 88.392) (width 0.25) (layer "F.Cu") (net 2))
 (segment (start 136.1333 91.3237) (end 139.065 88.392) (width 0.25) (layer "F.Cu") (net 2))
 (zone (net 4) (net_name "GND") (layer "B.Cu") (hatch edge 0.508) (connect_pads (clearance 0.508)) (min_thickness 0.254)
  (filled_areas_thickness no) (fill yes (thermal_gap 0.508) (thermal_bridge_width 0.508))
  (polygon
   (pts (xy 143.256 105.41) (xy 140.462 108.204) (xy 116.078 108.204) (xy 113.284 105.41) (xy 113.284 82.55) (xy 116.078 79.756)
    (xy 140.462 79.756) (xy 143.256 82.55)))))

